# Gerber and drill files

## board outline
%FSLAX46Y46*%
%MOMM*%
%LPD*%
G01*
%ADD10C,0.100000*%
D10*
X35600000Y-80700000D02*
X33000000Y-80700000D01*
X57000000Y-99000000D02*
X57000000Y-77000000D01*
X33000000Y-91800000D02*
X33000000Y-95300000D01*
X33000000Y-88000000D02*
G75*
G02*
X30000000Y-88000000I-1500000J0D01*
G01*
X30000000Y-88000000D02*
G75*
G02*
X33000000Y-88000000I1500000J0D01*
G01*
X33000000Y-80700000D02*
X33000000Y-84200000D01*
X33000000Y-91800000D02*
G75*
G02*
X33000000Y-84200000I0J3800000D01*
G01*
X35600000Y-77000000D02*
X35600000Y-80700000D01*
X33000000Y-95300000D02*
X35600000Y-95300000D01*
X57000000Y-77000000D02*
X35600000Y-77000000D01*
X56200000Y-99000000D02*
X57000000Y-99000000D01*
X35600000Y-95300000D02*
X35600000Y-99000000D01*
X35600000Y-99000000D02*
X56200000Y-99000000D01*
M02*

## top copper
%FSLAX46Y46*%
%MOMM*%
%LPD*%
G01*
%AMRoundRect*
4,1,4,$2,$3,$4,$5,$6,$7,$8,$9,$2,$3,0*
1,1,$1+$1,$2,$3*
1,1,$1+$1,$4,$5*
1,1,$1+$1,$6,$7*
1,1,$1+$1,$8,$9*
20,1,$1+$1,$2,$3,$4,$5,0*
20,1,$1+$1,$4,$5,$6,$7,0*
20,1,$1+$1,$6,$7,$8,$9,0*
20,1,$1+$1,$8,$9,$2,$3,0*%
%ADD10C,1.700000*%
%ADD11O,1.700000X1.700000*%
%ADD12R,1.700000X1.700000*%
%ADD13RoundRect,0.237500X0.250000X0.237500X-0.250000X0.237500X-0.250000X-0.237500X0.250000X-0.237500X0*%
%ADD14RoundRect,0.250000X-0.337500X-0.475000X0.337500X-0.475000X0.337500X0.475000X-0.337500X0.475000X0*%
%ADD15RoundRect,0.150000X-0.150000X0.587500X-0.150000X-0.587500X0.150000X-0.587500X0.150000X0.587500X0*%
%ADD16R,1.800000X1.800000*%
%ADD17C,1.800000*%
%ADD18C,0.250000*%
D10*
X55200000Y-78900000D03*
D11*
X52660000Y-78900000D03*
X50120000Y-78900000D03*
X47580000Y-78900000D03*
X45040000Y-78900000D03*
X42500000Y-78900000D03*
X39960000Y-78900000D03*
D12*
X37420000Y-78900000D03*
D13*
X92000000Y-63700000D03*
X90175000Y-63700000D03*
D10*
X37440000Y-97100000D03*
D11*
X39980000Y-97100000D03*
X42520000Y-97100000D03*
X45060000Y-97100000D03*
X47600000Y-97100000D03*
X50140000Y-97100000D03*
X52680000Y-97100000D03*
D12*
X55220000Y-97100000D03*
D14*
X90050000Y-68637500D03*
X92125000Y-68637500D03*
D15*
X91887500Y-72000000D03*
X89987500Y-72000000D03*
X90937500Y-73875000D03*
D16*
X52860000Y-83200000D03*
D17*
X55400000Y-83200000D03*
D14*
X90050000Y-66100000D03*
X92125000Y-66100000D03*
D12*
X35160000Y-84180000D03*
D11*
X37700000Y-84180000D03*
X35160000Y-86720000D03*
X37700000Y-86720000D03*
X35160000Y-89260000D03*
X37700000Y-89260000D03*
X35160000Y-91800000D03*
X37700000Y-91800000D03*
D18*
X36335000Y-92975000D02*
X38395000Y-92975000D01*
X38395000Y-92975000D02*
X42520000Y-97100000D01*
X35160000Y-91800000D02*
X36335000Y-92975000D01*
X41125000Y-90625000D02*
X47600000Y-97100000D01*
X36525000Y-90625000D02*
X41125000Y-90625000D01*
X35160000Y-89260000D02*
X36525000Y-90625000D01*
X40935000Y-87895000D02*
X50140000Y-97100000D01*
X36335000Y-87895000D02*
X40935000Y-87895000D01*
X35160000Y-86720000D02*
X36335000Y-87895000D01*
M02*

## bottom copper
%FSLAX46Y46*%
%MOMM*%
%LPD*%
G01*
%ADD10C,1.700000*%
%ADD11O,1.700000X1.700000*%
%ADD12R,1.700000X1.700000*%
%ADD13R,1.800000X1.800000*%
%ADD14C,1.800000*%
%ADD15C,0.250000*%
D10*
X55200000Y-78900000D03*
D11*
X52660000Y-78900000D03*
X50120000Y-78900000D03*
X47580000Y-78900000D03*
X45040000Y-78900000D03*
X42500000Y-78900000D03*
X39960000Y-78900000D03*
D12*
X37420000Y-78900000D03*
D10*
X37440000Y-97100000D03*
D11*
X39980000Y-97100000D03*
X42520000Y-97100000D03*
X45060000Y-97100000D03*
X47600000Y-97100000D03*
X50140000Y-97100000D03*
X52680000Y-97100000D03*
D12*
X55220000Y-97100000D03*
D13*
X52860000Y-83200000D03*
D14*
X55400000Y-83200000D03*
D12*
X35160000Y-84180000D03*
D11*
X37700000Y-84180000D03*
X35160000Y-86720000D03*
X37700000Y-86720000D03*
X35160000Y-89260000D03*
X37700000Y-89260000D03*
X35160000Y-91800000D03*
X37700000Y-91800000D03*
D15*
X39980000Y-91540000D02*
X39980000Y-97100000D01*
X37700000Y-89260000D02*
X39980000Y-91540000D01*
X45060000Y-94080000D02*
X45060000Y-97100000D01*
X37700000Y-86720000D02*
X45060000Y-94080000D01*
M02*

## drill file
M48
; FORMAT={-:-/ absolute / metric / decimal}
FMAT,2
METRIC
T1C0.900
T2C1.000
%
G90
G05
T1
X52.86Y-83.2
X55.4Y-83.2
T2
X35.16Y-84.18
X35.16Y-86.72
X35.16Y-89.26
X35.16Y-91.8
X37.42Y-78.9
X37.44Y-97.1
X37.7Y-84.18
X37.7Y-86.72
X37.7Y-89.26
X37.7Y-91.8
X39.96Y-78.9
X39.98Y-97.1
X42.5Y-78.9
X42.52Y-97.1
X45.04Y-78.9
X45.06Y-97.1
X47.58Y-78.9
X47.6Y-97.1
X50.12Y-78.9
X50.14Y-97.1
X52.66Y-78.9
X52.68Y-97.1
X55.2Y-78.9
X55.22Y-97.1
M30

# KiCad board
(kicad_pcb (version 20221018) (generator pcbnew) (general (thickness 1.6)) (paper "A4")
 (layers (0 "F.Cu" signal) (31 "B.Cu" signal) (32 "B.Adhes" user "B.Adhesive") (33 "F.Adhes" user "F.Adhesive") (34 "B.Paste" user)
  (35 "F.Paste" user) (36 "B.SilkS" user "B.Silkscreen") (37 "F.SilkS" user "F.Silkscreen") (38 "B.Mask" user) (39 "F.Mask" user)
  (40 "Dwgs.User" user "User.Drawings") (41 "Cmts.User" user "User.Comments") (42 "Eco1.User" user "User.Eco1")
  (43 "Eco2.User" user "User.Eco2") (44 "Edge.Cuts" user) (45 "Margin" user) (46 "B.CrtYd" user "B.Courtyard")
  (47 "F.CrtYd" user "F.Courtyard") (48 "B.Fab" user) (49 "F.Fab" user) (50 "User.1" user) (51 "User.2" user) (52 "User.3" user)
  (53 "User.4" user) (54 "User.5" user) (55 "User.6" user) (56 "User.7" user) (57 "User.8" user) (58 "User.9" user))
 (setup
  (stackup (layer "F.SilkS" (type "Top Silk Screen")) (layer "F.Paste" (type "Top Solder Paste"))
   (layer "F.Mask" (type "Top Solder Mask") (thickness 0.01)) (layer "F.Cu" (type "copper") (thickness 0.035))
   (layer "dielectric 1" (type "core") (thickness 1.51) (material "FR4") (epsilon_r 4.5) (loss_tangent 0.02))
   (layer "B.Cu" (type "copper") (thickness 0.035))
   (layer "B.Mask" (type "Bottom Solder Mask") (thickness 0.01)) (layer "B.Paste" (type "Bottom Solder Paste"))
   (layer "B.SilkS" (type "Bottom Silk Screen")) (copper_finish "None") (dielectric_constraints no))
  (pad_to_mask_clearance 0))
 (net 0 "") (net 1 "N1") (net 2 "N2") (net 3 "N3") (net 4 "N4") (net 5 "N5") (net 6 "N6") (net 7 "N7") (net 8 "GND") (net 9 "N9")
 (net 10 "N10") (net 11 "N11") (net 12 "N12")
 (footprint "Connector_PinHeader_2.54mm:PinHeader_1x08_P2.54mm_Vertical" (layer "F.Cu") (at 55.2 78.9 -90)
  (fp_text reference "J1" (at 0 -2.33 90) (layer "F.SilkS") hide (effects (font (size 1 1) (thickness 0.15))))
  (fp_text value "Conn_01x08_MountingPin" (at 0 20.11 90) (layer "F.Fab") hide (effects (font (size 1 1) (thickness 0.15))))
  (pad "1" thru_hole circle (at 0 0 270) (size 1.7 1.7) (drill 1) (layers "*.Cu" "*.Mask") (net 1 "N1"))
  (pad "2" thru_hole oval (at 0 2.54 270) (size 1.7 1.7) (drill 1) (layers "*.Cu" "*.Mask") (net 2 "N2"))
  (pad "3" thru_hole oval (at 0 5.08 270) (size 1.7 1.7) (drill 1) (layers "*.Cu" "*.Mask") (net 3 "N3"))
  (pad "4" thru_hole oval (at 0 7.62 270) (size 1.7 1.7) (drill 1) (layers "*.Cu" "*.Mask") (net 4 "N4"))
  (pad "5" thru_hole oval (at 0 10.16 270) (size 1.7 1.7) (drill 1) (layers "*.Cu" "*.Mask") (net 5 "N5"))
  (pad "6" thru_hole oval (at 0 12.7 270) (size 1.7 1.7) (drill 1) (layers "*.Cu" "*.Mask") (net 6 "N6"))
  (pad "7" thru_hole oval (at 0 15.24 270) (size 1.7 1.7) (drill 1) (layers "*.Cu" "*.Mask") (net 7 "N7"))
  (pad "8" thru_hole rect (at 0 17.78 270) (size 1.7 1.7) (drill 1) (layers "*.Cu" "*.Mask") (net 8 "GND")))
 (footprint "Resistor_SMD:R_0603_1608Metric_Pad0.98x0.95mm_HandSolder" (layer "F.Cu") (at 91.0875 63.7 180)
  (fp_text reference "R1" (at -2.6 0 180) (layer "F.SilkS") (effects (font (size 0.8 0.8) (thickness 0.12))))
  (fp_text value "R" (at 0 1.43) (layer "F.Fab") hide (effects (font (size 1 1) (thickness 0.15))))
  (pad "1" smd roundrect (at -0.9125 0 180) (size 0.975 0.95) (layers "F.Cu" "F.Paste" "F.Mask") (roundrect_rratio 0.25) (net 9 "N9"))
  (pad "2" smd roundrect (at 0.9125 0 180) (size 0.975 0.95) (layers "F.Cu" "F.Paste" "F.Mask") (roundrect_rratio 0.25) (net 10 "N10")))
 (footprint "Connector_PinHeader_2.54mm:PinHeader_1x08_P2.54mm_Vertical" (layer "F.Cu") (at 37.44 97.1 90)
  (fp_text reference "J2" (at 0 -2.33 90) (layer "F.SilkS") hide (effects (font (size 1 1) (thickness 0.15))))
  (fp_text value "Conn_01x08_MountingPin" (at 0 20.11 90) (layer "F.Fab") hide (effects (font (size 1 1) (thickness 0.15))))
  (pad "1" thru_hole circle (at 0 0 90) (size 1.7 1.7) (drill 1) (layers "*.Cu" "*.Mask") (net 1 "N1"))
  (pad "2" thru_hole oval (at 0 2.54 90) (size 1.7 1.7) (drill 1) (layers "*.Cu" "*.Mask") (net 2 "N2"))
  (pad "3" thru_hole oval (at 0 5.08 90) (size 1.7 1.7) (drill 1) (layers "*.Cu" "*.Mask") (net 3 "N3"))
  (pad "4" thru_hole oval (at 0 7.62 90) (size 1.7 1.7) (drill 1) (layers "*.Cu" "*.Mask") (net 4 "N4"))
  (pad "5" thru_hole oval (at 0 10.16 90) (size 1.7 1.7) (drill 1) (layers "*.Cu" "*.Mask") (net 5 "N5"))
  (pad "6" thru_hole oval (at 0 12.7 90) (size 1.7 1.7) (drill 1) (layers "*.Cu" "*.Mask") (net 6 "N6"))
  (pad "7" thru_hole oval (at 0 15.24 90) (size 1.7 1.7) (drill 1) (layers "*.Cu" "*.Mask") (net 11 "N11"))
  (pad "8" thru_hole rect (at 0 17.78 90) (size 1.7 1.7) (drill 1) (layers "*.Cu" "*.Mask") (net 8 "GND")))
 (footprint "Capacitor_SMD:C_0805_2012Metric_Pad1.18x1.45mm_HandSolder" (layer "F.Cu") (at 91.0875 68.6375)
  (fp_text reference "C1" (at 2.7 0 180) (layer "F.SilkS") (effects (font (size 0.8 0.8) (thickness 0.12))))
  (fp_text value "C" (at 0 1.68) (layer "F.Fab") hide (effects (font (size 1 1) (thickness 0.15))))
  (pad "1" smd roundrect (at -1.0375 0) (size 1.175 1.45) (layers "F.Cu" "F.Paste" "F.Mask") (roundrect_rratio 0.2127659574) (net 10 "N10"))
  (pad "2" smd roundrect (at 1.0375 0) (size 1.175 1.45) (layers "F.Cu" "F.Paste" "F.Mask") (roundrect_rratio 0.2127659574) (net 8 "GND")))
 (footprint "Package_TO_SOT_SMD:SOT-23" (layer "F.Cu") (at 90.9375 72.9375 -90)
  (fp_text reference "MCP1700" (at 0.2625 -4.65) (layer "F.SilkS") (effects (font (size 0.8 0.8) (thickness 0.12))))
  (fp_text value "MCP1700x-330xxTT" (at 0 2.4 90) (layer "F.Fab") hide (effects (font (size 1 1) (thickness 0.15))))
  (pad "1" smd roundrect (at -0.9375 -0.95 270) (size 1.475 0.6) (layers "F.Cu" "F.Paste" "F.Mask") (roundrect_rratio 0.25) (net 8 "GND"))
  (pad "2" smd roundrect (at -0.9375 0.95 270) (size 1.475 0.6) (layers "F.Cu" "F.Paste" "F.Mask") (roundrect_rratio 0.25) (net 10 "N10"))
  (pad "3" smd roundrect (at 0.9375 0 270) (size 1.475 0.6) (layers "F.Cu" "F.Paste" "F.Mask") (roundrect_rratio 0.25) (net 1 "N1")))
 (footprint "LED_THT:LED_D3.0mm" (layer "F.Cu") (at 52.86 83.2)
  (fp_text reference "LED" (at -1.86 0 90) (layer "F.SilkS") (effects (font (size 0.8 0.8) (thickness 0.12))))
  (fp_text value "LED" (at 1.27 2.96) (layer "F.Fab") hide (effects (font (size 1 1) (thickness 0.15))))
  (pad "1" thru_hole rect (at 0 0) (size 1.8 1.8) (drill 0.9) (layers "*.Cu" "*.Mask") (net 8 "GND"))
  (pad "2" thru_hole circle (at 2.54 0) (size 1.8 1.8) (drill 0.9) (layers "*.Cu" "*.Mask") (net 9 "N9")))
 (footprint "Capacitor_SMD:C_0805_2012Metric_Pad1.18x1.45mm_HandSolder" (layer "F.Cu") (at 91.0875 66.1)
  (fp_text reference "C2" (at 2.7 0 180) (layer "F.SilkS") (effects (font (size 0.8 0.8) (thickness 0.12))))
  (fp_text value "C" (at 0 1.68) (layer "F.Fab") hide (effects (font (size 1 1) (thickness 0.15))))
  (pad "1" smd roundrect (at -1.0375 0) (size 1.175 1.45) (layers "F.Cu" "F.Paste" "F.Mask") (roundrect_rratio 0.2127659574) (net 10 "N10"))
  (pad "2" smd roundrect (at 1.0375 0) (size 1.175 1.45) (layers "F.Cu" "F.Paste" "F.Mask") (roundrect_rratio 0.2127659574) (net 8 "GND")))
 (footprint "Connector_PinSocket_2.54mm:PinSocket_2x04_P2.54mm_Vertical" (layer "B.Cu") (at 35.16 84.18 180)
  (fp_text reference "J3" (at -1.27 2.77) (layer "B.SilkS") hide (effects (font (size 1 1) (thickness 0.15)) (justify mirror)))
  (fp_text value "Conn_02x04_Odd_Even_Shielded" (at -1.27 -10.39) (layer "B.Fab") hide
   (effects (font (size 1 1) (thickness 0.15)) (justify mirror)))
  (pad "1" thru_hole rect (at 0 0 180) (size 1.7 1.7) (drill 1) (layers "*.Cu" "*.Mask") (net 8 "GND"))
  (pad "2" thru_hole oval (at -2.54 0 180) (size 1.7 1.7) (drill 1) (layers "*.Cu" "*.Mask") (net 10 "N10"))
  (pad "3" thru_hole oval (at 0 -2.54 180) (size 1.7 1.7) (drill 1) (layers "*.Cu" "*.Mask") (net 6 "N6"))
  (pad "4" thru_hole oval (at -2.54 -2.54 180) (size 1.7 1.7) (drill 1) (layers "*.Cu" "*.Mask") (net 4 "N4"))
  (pad "5" thru_hole oval (at 0 -5.08 180) (size 1.7 1.7) (drill 1) (layers "*.Cu" "*.Mask") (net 5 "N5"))
  (pad "6" thru_hole oval (at -2.54 -5.08 180) (size 1.7 1.7) (drill 1) (layers "*.Cu" "*.Mask") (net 2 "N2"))
  (pad "7" thru_hole oval (at 0 -7.62 180) (size 1.7 1.7) (drill 1) (layers "*.Cu" "*.Mask") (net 3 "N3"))
  (pad "8" thru_hole oval (at -2.54 -7.62 180) (size 1.7 1.7) (drill 1) (layers "*.Cu" "*.Mask") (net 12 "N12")))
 (gr_line (start 35.6 80.7) (end 33 80.7) (stroke (width 0.1) (type default)) (layer "Edge.Cuts"))
 (gr_line (start 57 99) (end 57 77) (stroke (width 0.1) (type default)) (layer "Edge.Cuts"))
 (gr_line (start 33 91.8) (end 33 95.3) (stroke (width 0.1) (type default)) (layer "Edge.Cuts"))
 (gr_circle (center 31.5 88) (end 33 88) (stroke (width 0.1) (type default)) (fill none) (layer "Edge.Cuts"))
 (gr_line (start 33 80.7) (end 33 84.2) (stroke (width 0.1) (type default)) (layer "Edge.Cuts"))
 (gr_arc (start 33 91.8) (mid 29.2 88) (end 33 84.2) (stroke (width 0.1) (type default)) (layer "Edge.Cuts"))
 (gr_line (start 35.6 77) (end 35.6 80.7) (stroke (width 0.1) (type default)) (layer "Edge.Cuts"))
 (gr_line (start 33 95.3) (end 35.6 95.3) (stroke (width 0.1) (type default)) (layer "Edge.Cuts"))
 (gr_line (start 57 77) (end 35.6 77) (stroke (width 0.1) (type default)) (layer "Edge.Cuts"))
 (gr_line (start 56.2 99) (end 57 99) (stroke (width 0.1) (type default)) (layer "Edge.Cuts"))
 (gr_line (start 35.6 95.3) (end 35.6 99) (stroke (width 0.1) (type default)) (layer "Edge.Cuts"))
 (gr_line (start 35.6 99) (end 56.2 99) (stroke (width 0.1) (type default)) (layer "Edge.Cuts"))
 (segment (start 39.98 91.54) (end 39.98 97.1) (width 0.25) (layer "B.Cu") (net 2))
 (segment (start 37.7 89.26) (end 39.98 91.54) (width 0.25) (layer "B.Cu") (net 2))
 (segment (start 36.335 92.975) (end 38.395 92.975) (width 0.25) (layer "F.Cu") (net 3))
 (segment (start 38.395 92.975) (end 42.52 97.1) (width 0.25) (layer "F.Cu") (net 3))
 (segment (start 35.16 91.8) (end 36.335 92.975) (width 0.25) (layer "F.Cu") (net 3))
 (segment (start 45.06 94.08) (end 45.06 97.1) (width 0.25) (layer "B.Cu") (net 4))
 (segment (start 37.7 86.72) (end 45.06 94.08) (width 0.25) (layer "B.Cu") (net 4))
 (segment (start 41.125 90.625) (end 47.6 97.1) (width 0.25) (layer "F.Cu") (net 5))
 (segment (start 36.525 90.625) (end 41.125 90.625) (width 0.25) (layer "F.Cu") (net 5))
 (segment (start 35.16 89.26) (end 36.525 90.625) (width 0.25) (layer "F.Cu") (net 5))
 (segment (start 40.935 87.895) (end 50.14 97.1) (width 0.25) (layer "F.Cu") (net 6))
 (segment (start 36.335 87.895) (end 40.935 87.895) (width 0.25) (layer "F.Cu") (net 6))
 (segment (start 35.16 86.72) (end 36.335 87.895) (width 0.25) (layer "F.Cu") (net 6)))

